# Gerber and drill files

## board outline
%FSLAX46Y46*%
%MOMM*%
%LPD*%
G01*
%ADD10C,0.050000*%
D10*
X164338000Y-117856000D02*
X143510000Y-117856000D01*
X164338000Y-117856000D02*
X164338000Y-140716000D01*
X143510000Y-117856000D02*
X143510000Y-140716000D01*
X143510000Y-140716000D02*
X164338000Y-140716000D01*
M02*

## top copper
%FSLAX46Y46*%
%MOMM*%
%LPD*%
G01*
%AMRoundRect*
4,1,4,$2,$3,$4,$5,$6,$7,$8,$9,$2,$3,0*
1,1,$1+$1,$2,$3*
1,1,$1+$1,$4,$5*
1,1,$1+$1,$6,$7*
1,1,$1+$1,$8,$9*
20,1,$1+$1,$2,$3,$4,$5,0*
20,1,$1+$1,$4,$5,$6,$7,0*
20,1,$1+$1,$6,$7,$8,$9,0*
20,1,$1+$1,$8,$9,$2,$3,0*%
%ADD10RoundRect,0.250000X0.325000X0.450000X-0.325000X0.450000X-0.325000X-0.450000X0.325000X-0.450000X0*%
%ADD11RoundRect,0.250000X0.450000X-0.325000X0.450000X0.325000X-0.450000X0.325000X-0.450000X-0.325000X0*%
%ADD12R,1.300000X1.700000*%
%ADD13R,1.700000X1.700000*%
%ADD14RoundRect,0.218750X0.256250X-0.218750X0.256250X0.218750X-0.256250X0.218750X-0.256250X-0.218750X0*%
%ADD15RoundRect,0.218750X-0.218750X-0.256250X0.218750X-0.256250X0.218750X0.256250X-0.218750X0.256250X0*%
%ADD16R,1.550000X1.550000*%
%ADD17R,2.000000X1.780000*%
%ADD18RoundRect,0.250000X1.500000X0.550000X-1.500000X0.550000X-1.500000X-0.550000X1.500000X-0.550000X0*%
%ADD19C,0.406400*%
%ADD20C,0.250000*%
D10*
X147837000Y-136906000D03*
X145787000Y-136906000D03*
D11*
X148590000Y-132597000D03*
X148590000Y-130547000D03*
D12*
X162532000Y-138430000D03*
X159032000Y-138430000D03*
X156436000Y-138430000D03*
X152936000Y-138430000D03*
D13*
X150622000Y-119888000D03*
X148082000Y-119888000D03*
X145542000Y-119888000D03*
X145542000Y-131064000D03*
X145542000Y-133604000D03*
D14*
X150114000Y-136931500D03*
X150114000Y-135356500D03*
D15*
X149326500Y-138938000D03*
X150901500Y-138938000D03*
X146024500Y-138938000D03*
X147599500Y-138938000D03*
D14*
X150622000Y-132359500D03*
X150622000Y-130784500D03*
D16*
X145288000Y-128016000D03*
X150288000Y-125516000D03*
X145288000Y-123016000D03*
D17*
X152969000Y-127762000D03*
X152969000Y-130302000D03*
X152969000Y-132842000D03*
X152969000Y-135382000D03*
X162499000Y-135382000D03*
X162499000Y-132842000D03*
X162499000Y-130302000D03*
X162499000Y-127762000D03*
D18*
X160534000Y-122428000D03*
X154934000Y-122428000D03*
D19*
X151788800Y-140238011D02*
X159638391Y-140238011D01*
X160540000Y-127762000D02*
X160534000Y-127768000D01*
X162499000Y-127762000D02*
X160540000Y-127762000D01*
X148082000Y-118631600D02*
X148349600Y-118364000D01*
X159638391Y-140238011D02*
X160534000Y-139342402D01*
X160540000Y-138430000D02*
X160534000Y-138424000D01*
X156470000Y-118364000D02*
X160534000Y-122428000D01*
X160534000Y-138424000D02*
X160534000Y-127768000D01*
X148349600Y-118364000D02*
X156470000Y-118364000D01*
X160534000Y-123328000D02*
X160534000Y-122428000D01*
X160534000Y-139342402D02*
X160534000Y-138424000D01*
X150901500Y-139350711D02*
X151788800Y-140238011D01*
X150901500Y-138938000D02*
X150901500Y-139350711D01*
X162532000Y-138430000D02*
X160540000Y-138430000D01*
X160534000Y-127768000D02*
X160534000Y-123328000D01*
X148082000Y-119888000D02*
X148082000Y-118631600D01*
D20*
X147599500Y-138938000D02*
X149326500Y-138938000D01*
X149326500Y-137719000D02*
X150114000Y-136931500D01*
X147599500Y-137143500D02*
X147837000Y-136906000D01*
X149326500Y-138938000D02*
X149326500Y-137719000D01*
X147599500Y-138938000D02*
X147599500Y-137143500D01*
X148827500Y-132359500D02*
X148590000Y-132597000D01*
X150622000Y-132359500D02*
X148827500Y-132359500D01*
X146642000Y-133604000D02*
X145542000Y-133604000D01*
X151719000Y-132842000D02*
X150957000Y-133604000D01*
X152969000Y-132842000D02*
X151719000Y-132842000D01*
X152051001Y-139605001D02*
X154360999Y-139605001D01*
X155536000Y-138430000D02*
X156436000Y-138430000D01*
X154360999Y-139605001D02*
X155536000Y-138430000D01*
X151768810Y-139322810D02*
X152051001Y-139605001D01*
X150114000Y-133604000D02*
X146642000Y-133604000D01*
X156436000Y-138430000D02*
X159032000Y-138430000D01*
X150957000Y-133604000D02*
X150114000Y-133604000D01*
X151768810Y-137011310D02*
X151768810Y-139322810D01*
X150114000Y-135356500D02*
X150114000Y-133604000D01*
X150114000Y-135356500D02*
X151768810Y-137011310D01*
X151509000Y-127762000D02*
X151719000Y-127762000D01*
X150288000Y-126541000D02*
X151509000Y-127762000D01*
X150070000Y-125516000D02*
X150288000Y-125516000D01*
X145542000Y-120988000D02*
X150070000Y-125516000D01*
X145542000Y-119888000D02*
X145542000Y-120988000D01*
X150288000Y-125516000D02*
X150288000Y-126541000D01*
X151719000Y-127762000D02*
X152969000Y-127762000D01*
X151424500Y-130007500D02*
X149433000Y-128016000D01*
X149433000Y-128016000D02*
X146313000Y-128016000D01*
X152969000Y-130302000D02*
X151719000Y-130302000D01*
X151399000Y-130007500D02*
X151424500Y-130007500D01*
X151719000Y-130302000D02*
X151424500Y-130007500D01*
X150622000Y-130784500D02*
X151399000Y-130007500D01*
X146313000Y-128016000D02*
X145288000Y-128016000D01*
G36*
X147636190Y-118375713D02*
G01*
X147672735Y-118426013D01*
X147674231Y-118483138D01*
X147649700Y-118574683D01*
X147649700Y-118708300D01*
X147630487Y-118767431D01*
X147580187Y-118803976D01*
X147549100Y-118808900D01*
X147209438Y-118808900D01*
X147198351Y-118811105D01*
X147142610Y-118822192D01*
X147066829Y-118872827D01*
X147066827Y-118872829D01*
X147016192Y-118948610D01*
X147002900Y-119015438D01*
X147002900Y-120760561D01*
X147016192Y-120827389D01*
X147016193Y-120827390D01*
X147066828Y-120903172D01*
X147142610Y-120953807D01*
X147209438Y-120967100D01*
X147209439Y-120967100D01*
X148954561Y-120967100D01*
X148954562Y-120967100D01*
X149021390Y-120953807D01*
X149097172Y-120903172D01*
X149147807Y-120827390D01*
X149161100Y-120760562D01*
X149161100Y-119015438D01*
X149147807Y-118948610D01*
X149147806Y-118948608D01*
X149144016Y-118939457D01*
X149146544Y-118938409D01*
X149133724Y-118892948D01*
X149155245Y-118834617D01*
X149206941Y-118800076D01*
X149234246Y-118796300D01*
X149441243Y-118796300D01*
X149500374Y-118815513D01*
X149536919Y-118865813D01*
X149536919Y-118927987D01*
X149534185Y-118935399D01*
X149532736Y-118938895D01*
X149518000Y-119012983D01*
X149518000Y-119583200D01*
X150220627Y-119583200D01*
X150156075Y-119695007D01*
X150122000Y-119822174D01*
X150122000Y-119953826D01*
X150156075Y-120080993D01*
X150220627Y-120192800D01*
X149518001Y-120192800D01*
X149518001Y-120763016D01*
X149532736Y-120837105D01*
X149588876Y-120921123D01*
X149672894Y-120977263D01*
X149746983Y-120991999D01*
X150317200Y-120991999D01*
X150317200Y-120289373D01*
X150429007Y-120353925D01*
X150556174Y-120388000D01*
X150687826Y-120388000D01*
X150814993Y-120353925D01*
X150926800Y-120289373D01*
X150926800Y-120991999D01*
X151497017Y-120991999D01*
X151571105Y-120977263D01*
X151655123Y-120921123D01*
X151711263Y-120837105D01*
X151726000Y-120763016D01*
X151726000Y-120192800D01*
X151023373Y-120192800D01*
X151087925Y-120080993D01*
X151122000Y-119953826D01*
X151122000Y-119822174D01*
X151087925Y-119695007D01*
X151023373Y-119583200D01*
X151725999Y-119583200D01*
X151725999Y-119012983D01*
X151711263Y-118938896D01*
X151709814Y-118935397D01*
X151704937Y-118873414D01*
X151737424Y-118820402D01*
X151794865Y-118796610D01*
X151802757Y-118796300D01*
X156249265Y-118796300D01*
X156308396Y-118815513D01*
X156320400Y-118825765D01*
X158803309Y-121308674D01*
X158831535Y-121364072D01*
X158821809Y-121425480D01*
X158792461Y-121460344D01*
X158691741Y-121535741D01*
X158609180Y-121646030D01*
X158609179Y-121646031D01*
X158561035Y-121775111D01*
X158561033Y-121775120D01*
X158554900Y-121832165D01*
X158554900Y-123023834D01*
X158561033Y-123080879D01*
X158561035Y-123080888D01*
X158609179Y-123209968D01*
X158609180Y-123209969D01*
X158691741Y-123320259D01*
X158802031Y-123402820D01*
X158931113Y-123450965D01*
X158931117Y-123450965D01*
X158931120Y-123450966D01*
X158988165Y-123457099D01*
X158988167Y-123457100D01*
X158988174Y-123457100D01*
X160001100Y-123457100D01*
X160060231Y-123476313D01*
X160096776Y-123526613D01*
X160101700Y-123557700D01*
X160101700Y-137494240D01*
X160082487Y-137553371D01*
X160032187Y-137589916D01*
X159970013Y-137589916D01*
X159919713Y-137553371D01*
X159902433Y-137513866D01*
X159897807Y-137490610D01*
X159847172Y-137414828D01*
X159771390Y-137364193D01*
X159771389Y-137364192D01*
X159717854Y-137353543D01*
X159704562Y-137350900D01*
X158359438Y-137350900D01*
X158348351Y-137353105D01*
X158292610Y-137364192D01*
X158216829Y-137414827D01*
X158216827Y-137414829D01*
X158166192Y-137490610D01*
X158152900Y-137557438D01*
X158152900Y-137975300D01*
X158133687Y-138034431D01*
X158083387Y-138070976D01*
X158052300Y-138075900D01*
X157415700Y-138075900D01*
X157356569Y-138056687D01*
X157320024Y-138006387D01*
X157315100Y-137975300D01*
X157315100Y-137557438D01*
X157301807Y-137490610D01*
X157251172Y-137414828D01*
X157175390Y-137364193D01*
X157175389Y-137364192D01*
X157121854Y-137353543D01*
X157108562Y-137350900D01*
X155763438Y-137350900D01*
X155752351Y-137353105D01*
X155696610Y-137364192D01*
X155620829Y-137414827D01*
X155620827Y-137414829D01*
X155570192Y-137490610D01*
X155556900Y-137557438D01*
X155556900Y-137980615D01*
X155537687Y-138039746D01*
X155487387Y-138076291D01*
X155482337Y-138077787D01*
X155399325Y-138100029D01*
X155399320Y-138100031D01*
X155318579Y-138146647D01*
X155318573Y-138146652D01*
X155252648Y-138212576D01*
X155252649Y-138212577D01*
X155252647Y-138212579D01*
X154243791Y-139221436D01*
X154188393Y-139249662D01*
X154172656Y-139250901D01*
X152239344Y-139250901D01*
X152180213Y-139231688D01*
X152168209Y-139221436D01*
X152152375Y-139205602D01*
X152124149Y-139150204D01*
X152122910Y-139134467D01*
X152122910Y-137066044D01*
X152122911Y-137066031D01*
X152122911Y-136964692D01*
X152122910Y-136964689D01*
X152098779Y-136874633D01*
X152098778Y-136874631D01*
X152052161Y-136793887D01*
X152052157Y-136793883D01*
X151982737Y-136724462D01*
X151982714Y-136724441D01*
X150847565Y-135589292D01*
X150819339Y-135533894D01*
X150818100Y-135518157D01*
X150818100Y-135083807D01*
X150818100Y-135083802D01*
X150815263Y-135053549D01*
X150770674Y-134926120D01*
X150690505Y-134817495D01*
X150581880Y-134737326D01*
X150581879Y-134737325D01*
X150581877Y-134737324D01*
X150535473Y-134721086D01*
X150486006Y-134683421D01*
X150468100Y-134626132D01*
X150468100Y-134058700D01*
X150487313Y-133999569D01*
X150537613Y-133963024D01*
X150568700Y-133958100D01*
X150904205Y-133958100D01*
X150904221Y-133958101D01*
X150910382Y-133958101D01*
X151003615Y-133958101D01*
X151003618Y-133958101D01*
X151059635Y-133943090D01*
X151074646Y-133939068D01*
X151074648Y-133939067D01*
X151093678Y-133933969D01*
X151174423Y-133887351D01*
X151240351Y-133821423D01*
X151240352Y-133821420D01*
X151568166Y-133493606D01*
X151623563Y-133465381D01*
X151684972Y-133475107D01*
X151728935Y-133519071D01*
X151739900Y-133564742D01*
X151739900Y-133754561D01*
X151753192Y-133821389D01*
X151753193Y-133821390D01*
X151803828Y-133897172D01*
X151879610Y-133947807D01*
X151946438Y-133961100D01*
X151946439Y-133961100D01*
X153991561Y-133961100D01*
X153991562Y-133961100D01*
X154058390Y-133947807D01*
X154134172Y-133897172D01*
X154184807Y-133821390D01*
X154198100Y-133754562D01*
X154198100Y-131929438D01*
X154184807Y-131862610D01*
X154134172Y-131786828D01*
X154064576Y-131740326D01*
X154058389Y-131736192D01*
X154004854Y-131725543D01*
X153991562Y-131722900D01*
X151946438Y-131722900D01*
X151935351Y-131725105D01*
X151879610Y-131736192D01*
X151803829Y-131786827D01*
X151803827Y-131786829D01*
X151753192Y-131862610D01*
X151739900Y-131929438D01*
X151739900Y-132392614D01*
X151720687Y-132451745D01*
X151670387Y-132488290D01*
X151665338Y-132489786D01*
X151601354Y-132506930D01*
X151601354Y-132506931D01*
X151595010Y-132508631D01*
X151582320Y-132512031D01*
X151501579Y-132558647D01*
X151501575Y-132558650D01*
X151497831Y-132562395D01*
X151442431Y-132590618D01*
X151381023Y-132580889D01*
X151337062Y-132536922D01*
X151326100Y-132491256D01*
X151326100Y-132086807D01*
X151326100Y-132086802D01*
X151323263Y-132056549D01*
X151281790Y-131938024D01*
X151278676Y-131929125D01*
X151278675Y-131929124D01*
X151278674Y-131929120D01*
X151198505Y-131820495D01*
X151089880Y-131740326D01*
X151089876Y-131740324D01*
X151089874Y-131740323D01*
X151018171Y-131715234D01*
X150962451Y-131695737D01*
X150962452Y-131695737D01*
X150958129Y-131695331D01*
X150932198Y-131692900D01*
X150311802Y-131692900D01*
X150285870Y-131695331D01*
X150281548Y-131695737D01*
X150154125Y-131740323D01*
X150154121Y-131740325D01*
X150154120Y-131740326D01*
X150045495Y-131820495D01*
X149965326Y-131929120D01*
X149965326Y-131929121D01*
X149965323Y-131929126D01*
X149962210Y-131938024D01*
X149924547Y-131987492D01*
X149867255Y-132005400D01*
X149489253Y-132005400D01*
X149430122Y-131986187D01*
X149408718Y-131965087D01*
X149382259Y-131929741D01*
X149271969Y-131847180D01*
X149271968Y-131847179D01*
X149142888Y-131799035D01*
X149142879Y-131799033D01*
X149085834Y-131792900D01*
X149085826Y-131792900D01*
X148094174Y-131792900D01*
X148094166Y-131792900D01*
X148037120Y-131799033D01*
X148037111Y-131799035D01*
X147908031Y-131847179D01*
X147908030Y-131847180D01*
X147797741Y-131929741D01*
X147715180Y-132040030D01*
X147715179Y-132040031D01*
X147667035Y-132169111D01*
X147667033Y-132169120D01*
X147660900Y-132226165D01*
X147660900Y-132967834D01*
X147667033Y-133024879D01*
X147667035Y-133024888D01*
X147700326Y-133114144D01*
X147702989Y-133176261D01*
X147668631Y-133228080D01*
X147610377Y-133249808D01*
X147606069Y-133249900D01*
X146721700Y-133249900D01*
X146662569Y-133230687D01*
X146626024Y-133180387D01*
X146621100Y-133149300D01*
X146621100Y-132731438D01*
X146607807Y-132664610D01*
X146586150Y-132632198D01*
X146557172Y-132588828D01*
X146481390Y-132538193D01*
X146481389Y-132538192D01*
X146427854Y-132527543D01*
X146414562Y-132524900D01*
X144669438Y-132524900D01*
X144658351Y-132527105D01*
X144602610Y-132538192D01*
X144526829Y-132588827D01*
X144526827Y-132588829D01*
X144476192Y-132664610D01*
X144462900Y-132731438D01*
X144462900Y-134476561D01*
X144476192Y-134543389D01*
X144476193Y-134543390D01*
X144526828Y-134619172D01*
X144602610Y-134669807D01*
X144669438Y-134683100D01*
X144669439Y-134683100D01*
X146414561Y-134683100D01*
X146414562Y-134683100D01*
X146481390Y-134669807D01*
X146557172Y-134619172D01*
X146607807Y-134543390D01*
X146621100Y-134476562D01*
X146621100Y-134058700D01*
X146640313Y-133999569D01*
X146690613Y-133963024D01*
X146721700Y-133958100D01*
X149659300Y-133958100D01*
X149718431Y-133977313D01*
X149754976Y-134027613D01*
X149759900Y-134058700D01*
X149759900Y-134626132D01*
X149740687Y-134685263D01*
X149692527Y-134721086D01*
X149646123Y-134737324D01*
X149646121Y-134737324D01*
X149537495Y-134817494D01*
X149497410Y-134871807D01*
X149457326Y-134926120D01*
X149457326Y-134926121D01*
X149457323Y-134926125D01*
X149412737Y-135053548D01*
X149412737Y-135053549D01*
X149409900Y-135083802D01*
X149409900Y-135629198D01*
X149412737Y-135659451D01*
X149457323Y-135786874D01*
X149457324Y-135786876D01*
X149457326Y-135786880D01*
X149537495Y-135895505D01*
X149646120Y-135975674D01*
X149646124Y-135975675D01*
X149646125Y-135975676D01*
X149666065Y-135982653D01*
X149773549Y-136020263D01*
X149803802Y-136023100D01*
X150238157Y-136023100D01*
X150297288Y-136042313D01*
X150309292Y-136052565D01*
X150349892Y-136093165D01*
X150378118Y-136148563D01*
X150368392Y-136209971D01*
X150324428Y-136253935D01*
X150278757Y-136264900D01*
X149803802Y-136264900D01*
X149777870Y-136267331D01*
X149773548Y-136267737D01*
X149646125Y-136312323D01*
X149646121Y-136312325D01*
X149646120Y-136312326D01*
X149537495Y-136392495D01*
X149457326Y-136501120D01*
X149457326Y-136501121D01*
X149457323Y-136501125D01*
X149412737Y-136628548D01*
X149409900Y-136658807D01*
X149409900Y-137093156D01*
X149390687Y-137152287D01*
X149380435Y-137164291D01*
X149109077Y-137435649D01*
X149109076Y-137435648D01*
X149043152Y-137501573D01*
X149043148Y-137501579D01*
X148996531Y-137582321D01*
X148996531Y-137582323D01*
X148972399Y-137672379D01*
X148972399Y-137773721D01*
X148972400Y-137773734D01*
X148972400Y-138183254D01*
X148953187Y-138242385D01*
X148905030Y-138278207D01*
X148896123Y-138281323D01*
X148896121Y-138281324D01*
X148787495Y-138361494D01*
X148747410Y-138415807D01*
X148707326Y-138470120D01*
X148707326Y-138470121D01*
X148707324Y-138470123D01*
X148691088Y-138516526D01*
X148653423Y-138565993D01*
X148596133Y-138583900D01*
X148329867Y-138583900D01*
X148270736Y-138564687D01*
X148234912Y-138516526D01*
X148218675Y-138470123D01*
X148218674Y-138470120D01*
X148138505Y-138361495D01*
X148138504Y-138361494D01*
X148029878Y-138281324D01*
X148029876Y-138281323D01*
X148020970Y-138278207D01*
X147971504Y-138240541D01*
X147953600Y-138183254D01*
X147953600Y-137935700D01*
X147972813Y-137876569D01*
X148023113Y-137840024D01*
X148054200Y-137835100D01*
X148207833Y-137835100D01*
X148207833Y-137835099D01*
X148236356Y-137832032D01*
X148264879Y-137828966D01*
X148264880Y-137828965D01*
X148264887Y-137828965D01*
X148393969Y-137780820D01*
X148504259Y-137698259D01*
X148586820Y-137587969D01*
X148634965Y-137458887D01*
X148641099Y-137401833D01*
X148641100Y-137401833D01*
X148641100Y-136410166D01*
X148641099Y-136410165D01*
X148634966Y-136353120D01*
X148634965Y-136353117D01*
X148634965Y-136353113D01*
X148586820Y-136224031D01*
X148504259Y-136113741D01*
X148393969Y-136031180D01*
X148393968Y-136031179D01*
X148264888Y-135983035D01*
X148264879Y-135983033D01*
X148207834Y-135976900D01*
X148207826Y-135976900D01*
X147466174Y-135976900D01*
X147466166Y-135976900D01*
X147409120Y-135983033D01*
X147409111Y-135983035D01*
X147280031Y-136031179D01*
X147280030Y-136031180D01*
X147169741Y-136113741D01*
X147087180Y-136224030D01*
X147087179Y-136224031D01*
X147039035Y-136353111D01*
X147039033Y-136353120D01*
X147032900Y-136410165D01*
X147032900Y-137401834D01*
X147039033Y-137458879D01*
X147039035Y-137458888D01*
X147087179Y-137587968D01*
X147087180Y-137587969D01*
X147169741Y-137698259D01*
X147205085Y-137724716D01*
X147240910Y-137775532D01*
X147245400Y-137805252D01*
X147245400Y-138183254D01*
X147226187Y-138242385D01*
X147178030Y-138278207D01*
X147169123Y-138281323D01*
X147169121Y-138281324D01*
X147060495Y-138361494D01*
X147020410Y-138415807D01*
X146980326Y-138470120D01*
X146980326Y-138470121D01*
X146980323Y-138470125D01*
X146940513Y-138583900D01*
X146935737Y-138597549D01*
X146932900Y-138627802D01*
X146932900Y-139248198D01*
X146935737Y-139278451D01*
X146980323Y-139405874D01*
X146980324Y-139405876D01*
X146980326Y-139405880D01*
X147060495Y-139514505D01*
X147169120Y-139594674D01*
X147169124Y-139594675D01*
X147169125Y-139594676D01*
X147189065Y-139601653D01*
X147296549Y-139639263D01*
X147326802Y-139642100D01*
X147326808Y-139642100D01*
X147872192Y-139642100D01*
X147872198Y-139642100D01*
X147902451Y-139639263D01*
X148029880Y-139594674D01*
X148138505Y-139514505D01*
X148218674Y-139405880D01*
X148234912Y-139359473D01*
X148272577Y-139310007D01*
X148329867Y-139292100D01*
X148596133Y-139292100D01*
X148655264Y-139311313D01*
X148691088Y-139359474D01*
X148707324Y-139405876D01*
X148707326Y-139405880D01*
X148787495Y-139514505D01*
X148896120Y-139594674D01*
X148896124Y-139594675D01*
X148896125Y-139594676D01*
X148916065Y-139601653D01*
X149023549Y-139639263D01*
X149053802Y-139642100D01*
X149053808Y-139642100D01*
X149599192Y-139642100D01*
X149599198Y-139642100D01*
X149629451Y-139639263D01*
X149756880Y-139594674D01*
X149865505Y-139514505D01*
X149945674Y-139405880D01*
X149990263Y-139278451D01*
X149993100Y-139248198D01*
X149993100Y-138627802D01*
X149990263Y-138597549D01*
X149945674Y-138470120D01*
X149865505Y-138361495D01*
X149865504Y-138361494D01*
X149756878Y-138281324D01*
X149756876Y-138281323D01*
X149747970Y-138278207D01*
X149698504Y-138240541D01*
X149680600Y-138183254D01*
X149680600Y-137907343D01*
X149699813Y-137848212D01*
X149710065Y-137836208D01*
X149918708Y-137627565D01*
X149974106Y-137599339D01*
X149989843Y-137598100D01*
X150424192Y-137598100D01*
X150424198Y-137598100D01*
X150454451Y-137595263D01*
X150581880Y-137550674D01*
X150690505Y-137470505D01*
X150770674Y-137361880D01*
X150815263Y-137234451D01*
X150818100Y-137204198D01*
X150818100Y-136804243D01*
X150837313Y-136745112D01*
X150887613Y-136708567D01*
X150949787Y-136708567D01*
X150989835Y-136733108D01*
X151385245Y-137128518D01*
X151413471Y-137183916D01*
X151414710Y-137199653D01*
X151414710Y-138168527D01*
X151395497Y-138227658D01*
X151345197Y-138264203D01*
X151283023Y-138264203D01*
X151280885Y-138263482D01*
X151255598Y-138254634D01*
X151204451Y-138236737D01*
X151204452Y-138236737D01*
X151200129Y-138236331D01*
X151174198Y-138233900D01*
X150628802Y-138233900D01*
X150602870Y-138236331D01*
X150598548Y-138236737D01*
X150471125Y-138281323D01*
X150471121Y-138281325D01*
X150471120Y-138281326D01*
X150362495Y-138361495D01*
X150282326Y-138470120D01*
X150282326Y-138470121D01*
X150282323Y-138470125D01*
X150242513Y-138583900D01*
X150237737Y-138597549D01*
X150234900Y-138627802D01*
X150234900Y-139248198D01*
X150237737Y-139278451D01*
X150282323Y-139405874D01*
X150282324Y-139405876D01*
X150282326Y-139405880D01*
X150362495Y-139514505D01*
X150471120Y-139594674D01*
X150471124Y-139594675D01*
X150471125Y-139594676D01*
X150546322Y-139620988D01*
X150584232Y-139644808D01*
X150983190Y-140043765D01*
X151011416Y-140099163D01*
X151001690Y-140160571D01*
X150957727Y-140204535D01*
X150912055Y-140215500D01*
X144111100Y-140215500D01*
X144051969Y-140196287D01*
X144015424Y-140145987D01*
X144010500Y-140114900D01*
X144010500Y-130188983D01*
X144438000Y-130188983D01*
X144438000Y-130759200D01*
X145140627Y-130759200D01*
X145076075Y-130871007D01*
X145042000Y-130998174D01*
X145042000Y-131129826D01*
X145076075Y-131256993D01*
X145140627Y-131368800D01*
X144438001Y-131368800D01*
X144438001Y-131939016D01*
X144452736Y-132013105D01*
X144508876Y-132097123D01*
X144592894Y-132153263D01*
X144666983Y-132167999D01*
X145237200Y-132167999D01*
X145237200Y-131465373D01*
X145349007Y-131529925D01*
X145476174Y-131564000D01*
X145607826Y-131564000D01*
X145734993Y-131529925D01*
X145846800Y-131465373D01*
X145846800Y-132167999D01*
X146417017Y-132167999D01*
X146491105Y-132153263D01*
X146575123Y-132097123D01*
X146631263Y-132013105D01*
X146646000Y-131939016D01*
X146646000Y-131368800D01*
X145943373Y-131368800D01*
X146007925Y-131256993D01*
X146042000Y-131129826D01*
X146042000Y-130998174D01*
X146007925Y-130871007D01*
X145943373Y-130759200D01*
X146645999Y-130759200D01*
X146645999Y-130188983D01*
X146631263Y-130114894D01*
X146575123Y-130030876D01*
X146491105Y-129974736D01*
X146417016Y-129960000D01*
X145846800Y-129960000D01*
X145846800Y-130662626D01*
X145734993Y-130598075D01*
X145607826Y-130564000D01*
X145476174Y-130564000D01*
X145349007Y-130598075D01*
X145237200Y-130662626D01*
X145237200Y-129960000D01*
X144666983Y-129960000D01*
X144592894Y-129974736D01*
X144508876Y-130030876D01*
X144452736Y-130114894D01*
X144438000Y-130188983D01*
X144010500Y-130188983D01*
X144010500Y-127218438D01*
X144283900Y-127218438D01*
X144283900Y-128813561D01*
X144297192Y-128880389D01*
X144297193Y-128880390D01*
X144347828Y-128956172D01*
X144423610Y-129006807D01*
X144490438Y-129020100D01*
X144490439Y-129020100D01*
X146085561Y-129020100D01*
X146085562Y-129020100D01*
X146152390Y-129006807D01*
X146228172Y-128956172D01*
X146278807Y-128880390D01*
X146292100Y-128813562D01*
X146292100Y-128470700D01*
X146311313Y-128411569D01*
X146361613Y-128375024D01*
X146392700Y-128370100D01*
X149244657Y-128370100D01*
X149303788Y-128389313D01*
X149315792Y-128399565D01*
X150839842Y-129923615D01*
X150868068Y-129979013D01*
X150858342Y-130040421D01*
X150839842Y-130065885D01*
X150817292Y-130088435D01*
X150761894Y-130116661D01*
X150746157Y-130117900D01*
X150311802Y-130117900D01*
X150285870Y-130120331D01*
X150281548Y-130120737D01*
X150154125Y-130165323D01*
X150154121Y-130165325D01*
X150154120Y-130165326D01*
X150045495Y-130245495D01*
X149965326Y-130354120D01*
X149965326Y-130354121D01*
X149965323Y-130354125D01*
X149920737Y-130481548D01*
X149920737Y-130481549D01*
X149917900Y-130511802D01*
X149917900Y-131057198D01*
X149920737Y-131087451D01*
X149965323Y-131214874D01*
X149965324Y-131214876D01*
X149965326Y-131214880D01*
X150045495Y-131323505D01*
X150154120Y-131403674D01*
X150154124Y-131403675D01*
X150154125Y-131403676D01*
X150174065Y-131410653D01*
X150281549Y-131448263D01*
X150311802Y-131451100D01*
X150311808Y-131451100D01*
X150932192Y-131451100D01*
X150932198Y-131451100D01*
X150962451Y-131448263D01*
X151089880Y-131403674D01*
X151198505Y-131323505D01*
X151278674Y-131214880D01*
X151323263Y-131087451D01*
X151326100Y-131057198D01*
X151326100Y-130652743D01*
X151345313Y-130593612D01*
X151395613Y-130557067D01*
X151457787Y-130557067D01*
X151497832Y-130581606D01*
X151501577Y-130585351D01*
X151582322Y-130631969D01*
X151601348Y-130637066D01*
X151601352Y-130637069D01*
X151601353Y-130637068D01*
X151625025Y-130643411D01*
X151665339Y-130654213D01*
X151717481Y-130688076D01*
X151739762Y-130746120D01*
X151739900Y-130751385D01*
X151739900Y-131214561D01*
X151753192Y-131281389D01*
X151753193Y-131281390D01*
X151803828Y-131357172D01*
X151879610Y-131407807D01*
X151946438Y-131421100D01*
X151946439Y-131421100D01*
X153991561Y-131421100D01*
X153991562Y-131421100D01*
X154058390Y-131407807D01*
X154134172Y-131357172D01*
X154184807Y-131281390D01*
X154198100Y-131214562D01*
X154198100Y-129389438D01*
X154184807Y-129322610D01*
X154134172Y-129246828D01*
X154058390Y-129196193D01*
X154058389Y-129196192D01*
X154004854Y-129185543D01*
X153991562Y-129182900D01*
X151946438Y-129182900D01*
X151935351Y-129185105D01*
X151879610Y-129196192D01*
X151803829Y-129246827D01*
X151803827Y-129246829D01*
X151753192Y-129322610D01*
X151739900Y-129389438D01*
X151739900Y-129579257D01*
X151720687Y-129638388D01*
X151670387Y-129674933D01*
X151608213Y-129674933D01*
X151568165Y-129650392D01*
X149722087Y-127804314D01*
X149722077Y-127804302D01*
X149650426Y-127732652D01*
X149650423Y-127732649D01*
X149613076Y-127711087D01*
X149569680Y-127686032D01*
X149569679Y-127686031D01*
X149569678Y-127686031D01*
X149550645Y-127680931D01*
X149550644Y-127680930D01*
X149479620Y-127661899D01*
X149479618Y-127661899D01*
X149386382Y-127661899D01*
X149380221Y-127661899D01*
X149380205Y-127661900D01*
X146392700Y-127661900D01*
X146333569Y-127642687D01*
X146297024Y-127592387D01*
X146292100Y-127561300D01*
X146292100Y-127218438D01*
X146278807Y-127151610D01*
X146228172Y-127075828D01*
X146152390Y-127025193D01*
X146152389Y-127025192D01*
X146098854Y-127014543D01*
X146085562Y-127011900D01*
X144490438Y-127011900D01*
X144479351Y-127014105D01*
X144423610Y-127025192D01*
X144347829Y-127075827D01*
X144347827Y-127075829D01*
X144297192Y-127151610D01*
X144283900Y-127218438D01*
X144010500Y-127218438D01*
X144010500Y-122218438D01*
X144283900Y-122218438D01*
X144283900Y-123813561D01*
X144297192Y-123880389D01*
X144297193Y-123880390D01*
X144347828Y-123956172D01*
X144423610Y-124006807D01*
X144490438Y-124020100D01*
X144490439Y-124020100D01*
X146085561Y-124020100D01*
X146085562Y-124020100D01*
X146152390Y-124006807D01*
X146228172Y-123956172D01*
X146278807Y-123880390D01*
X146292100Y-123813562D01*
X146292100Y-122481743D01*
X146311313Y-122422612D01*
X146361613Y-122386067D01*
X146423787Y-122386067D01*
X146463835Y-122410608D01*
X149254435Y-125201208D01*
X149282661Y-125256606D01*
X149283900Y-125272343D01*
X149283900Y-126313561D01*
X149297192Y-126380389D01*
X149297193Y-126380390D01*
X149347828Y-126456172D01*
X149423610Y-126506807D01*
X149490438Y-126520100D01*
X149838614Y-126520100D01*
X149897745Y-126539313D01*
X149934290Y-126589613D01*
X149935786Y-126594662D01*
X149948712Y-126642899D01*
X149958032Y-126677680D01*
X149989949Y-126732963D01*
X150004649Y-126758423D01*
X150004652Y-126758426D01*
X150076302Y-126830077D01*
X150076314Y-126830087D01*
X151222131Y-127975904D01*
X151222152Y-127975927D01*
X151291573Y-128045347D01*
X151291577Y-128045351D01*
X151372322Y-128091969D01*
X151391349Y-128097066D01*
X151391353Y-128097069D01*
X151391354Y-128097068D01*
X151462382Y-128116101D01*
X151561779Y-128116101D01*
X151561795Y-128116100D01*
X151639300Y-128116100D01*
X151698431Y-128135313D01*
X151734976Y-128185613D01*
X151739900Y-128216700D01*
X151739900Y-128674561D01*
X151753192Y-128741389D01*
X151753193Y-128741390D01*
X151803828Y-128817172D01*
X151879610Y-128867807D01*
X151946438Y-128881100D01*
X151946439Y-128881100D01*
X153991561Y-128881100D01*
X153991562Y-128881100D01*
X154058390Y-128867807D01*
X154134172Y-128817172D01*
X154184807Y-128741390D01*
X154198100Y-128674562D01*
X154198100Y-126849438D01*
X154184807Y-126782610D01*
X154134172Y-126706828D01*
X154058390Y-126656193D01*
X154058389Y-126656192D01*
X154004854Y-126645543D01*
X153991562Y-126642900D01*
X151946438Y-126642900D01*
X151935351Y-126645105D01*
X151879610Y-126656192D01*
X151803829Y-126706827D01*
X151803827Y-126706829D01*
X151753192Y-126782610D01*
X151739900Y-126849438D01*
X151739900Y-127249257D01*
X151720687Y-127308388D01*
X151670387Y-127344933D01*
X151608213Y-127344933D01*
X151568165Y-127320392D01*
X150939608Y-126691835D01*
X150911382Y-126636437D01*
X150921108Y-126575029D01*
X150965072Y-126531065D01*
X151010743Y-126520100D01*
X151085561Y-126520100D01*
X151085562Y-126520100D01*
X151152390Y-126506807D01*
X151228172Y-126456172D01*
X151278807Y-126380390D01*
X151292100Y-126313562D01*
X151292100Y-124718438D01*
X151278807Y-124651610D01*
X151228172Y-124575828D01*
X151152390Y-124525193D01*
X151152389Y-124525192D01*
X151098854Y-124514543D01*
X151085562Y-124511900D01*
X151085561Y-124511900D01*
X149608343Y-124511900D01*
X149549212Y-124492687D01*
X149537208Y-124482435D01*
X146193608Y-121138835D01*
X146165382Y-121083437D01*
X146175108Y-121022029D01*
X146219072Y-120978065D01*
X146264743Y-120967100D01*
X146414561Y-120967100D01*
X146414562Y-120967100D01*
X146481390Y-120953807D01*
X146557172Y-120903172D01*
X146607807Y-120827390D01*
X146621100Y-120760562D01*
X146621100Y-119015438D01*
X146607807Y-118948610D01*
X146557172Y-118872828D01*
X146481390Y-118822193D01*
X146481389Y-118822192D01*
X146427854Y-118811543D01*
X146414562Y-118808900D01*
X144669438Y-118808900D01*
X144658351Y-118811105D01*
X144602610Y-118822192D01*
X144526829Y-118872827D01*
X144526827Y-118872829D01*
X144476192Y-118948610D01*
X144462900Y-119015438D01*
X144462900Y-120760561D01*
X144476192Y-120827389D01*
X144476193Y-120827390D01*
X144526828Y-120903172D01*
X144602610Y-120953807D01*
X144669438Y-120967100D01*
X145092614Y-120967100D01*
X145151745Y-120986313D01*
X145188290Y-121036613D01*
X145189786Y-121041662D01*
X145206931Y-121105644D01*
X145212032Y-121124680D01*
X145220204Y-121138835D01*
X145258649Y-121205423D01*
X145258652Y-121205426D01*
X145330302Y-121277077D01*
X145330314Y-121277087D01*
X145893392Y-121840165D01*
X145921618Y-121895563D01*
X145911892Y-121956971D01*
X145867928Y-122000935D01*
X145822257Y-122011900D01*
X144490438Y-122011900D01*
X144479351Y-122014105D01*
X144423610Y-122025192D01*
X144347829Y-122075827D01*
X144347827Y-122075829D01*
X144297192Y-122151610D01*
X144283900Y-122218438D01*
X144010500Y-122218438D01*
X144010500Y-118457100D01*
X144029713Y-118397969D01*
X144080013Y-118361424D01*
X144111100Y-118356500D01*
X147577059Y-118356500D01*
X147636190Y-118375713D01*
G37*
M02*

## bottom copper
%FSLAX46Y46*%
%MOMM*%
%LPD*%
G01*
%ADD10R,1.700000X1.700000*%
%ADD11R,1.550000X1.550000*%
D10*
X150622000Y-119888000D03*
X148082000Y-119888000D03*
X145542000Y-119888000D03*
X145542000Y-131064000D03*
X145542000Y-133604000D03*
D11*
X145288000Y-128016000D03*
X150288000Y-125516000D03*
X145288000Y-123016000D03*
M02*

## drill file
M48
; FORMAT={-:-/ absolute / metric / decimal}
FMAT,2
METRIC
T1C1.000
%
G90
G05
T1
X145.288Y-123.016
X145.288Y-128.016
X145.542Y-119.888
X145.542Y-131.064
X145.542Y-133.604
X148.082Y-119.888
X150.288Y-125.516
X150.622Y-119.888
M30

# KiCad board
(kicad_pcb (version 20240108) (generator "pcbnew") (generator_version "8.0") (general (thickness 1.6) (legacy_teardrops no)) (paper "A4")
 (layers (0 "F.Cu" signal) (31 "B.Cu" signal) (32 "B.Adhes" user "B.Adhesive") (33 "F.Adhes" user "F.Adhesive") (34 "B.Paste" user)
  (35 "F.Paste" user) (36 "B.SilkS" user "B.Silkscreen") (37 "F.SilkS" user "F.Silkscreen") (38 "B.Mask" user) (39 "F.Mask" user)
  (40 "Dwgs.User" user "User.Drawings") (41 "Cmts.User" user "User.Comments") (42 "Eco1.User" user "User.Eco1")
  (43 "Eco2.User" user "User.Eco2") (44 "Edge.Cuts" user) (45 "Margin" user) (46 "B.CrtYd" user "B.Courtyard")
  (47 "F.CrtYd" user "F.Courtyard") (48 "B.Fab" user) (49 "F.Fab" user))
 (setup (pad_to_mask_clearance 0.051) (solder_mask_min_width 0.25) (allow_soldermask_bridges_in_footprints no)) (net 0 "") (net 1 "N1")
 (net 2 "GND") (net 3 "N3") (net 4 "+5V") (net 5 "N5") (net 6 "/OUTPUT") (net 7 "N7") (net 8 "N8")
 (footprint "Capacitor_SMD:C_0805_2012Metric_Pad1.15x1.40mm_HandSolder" (layer "F.Cu") (at 146.812 136.906 180)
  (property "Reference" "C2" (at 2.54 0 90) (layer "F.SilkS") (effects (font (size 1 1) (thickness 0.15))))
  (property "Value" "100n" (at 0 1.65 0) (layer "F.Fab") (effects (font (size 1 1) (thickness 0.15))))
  (pad "1" smd roundrect (at -1.025 0 180) (size 1.15 1.4) (layers "F.Cu" "F.Paste" "F.Mask") (roundrect_rratio 0.217391) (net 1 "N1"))
  (pad "2" smd roundrect (at 1.025 0 180) (size 1.15 1.4) (layers "F.Cu" "F.Paste" "F.Mask") (roundrect_rratio 0.217391) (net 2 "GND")))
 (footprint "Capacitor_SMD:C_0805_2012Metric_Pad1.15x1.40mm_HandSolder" (layer "F.Cu") (at 148.59 131.572 90)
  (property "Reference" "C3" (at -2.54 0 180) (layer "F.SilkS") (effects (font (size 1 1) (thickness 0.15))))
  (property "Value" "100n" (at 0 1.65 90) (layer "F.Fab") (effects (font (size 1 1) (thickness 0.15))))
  (pad "1" smd roundrect (at -1.025 0 90) (size 1.15 1.4) (layers "F.Cu" "F.Paste" "F.Mask") (roundrect_rratio 0.217391) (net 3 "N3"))
  (pad "2" smd roundrect (at 1.025 0 90) (size 1.15 1.4) (layers "F.Cu" "F.Paste" "F.Mask") (roundrect_rratio 0.217391) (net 2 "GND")))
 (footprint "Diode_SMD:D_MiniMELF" (layer "F.Cu") (at 160.782 138.43 180)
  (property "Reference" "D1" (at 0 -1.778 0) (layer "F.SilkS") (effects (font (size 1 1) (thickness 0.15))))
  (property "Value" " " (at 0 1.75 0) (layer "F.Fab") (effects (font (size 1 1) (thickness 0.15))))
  (pad "1" smd rect (at -1.75 0 180) (size 1.3 1.7) (layers "F.Cu" "F.Paste" "F.Mask") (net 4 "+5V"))
  (pad "2" smd rect (at 1.75 0 180) (size 1.3 1.7) (layers "F.Cu" "F.Paste" "F.Mask") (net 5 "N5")))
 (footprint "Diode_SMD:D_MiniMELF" (layer "F.Cu") (at 154.686 138.43 180)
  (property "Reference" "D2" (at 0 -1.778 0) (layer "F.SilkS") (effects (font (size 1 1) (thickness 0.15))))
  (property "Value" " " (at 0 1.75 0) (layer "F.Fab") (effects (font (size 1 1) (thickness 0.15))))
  (pad "1" smd rect (at -1.75 0 180) (size 1.3 1.7) (layers "F.Cu" "F.Paste" "F.Mask") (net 5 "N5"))
  (pad "2" smd rect (at 1.75 0 180) (size 1.3 1.7) (layers "F.Cu" "F.Paste" "F.Mask") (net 2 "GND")))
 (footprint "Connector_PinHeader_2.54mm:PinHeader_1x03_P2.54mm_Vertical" (layer "F.Cu") (at 150.622 119.888 -90)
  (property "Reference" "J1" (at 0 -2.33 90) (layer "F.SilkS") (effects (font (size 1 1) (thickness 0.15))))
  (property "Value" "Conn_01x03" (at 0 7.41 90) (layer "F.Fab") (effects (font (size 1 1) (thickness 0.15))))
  (pad "1" thru_hole rect (at 0 0 270) (size 1.7 1.7) (drill 1) (layers "*.Cu" "*.Mask") (remove_unused_layers no) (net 2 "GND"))
  (pad "2" thru_hole rect (at 0 2.54 270) (size 1.7 1.7) (drill 1) (layers "*.Cu" "*.Mask") (remove_unused_layers no) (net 4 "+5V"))
  (pad "3" thru_hole rect (at 0 5.08 270) (size 1.7 1.7) (drill 1) (layers "*.Cu" "*.Mask") (remove_unused_layers no) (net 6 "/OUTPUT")))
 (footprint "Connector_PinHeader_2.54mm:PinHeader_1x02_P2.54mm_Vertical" (layer "F.Cu") (at 145.542 131.064)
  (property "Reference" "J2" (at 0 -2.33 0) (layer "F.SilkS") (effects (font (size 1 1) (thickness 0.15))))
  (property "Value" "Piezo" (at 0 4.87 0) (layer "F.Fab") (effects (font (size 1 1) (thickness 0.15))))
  (pad "1" thru_hole rect (at 0 0) (size 1.7 1.7) (drill 1) (layers "*.Cu" "*.Mask") (remove_unused_layers no) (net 2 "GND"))
  (pad "2" thru_hole rect (at 0 2.54) (size 1.7 1.7) (drill 1) (layers "*.Cu" "*.Mask") (remove_unused_layers no) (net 5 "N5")))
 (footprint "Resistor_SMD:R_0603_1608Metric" (layer "F.Cu") (at 150.114 136.144 90)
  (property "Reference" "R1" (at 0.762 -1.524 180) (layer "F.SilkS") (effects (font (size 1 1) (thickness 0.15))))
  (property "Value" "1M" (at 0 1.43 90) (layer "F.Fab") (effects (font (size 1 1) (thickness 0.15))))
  (pad "1" smd roundrect (at -0.7875 0 90) (size 0.875 0.95) (layers "F.Cu" "F.Paste" "F.Mask") (roundrect_rratio 0.25) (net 1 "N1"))
  (pad "2" smd roundrect (at 0.7875 0 90) (size 0.875 0.95) (layers "F.Cu" "F.Paste" "F.Mask") (roundrect_rratio 0.25) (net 5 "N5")))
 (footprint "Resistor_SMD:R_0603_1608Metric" (layer "F.Cu") (at 150.114 138.938)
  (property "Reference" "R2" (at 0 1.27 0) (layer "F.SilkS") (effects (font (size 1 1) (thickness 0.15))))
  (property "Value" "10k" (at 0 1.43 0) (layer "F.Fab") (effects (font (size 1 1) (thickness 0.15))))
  (pad "1" smd roundrect (at -0.7875 0) (size 0.875 0.95) (layers "F.Cu" "F.Paste" "F.Mask") (roundrect_rratio 0.25) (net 1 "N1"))
  (pad "2" smd roundrect (at 0.7875 0) (size 0.875 0.95) (layers "F.Cu" "F.Paste" "F.Mask") (roundrect_rratio 0.25) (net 4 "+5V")))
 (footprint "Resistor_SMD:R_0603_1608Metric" (layer "F.Cu") (at 146.812 138.938)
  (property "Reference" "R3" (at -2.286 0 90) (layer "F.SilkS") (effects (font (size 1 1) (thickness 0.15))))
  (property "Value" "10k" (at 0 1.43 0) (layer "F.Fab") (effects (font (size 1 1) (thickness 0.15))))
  (pad "1" smd roundrect (at -0.7875 0) (size 0.875 0.95) (layers "F.Cu" "F.Paste" "F.Mask") (roundrect_rratio 0.25) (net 2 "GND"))
  (pad "2" smd roundrect (at 0.7875 0) (size 0.875 0.95) (layers "F.Cu" "F.Paste" "F.Mask") (roundrect_rratio 0.25) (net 1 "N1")))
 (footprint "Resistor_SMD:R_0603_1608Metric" (layer "F.Cu") (at 150.622 131.572 90)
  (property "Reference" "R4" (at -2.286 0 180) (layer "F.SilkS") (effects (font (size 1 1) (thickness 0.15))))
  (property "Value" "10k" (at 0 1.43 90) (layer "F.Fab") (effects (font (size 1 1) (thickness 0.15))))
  (pad "1" smd roundrect (at -0.7875 0 90) (size 0.875 0.95) (layers "F.Cu" "F.Paste" "F.Mask") (roundrect_rratio 0.25) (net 3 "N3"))
  (pad "2" smd roundrect (at 0.7875 0 90) (size 0.875 0.95) (layers "F.Cu" "F.Paste" "F.Mask") (roundrect_rratio 0.25) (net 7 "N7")))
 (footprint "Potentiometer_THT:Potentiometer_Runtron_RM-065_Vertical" (layer "F.Cu") (at 145.288 128.016 90)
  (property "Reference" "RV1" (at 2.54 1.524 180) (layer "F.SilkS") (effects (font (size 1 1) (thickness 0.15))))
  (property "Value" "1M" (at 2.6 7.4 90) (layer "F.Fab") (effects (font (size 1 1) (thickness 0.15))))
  (pad "1" thru_hole rect (at 0 0 90) (size 1.55 1.55) (drill 1) (layers "*.Cu" "*.Mask") (remove_unused_layers no) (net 7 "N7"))
  (pad "2" thru_hole rect (at 2.5 5 90) (size 1.55 1.55) (drill 1) (layers "*.Cu" "*.Mask") (remove_unused_layers no) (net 6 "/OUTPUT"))
  (pad "3" thru_hole rect (at 5 0 90) (size 1.55 1.55) (drill 1) (layers "*.Cu" "*.Mask") (remove_unused_layers no) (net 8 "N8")))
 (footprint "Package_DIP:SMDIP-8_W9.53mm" (layer "F.Cu") (at 157.734 131.572)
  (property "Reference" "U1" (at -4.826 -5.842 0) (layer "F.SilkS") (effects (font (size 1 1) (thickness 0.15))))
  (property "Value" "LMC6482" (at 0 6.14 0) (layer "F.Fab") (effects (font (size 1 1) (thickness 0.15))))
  (pad "1" smd rect (at -4.765 -3.81) (size 2 1.78) (layers "F.Cu" "F.Paste" "F.Mask") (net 6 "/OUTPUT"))
  (pad "2" smd rect (at -4.765 -1.27) (size 2 1.78) (layers "F.Cu" "F.Paste" "F.Mask") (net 7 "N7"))
  (pad "3" smd rect (at -4.765 1.27) (size 2 1.78) (layers "F.Cu" "F.Paste" "F.Mask") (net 5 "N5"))
  (pad "4" smd rect (at -4.765 3.81) (size 2 1.78) (layers "F.Cu" "F.Paste" "F.Mask") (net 2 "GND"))
  (pad "5" smd rect (at 4.765 3.81) (size 2 1.78) (layers "F.Cu" "F.Paste" "F.Mask"))
  (pad "6" smd rect (at 4.765 1.27) (size 2 1.78) (layers "F.Cu" "F.Paste" "F.Mask"))
  (pad "7" smd rect (at 4.765 -1.27) (size 2 1.78) (layers "F.Cu" "F.Paste" "F.Mask"))
  (pad "8" smd rect (at 4.765 -3.81) (size 2 1.78) (layers "F.Cu" "F.Paste" "F.Mask") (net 4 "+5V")))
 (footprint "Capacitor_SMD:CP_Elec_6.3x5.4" (layer "F.Cu") (at 157.734 122.428 180)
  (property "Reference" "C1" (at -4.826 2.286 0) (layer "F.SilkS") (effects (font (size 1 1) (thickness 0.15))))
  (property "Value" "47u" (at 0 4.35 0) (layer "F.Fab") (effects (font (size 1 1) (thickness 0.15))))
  (pad "1" smd roundrect (at -2.8 0 180) (size 3.5 1.6) (layers "F.Cu" "F.Paste" "F.Mask") (roundrect_rratio 0.15625) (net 4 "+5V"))
  (pad "2" smd roundrect (at 2.8 0 180) (size 3.5 1.6) (layers "F.Cu" "F.Paste" "F.Mask") (roundrect_rratio 0.15625) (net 2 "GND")))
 (gr_line (start 164.338 117.856) (end 143.51 117.856) (stroke (width 0.05) (type solid)) (layer "Edge.Cuts"))
 (gr_line (start 164.338 117.856) (end 164.338 140.716) (stroke (width 0.05) (type solid)) (layer "Edge.Cuts"))
 (gr_line (start 143.51 117.856) (end 143.51 140.716) (stroke (width 0.05) (type solid)) (layer "Edge.Cuts"))
 (gr_line (start 143.51 140.716) (end 164.338 140.716) (stroke (width 0.05) (type solid)) (layer "Edge.Cuts"))
 (segment (start 151.7888 140.238011) (end 159.638391 140.238011) (width 0.4064) (layer "F.Cu") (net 4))
 (segment (start 160.54 127.762) (end 160.534 127.768) (width 0.4064) (layer "F.Cu") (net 4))
 (segment (start 162.499 127.762) (end 160.54 127.762) (width 0.4064) (layer "F.Cu") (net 4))
 (segment (start 148.082 118.6316) (end 148.3496 118.364) (width 0.4064) (layer "F.Cu") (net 4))
 (segment (start 159.638391 140.238011) (end 160.534 139.342402) (width 0.4064) (layer "F.Cu") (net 4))
 (segment (start 160.54 138.43) (end 160.534 138.424) (width 0.4064) (layer "F.Cu") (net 4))
 (segment (start 156.47 118.364) (end 160.534 122.428) (width 0.4064) (layer "F.Cu") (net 4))
 (segment (start 160.534 138.424) (end 160.534 127.768) (width 0.4064) (layer "F.Cu") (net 4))
 (segment (start 148.3496 118.364) (end 156.47 118.364) (width 0.4064) (layer "F.Cu") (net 4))
 (segment (start 160.534 123.328) (end 160.534 122.428) (width 0.4064) (layer "F.Cu") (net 4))
 (segment (start 160.534 139.342402) (end 160.534 138.424) (width 0.4064) (layer "F.Cu") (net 4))
 (segment (start 150.9015 139.350711) (end 151.7888 140.238011) (width 0.4064) (layer "F.Cu") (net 4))
 (segment (start 150.9015 138.938) (end 150.9015 139.350711) (width 0.4064) (layer "F.Cu") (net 4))
 (segment (start 162.532 138.43) (end 160.54 138.43) (width 0.4064) (layer "F.Cu") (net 4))
 (segment (start 160.534 127.768) (end 160.534 123.328) (width 0.4064) (layer "F.Cu") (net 4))
 (segment (start 148.082 119.888) (end 148.082 118.6316) (width 0.4064) (layer "F.Cu") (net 4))
 (segment (start 147.5995 138.938) (end 149.3265 138.938) (width 0.25) (layer "F.Cu") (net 1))
 (segment (start 149.3265 137.719) (end 150.114 136.9315) (width 0.25) (layer "F.Cu") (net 1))
 (segment (start 147.5995 137.1435) (end 147.837 136.906) (width 0.25) (layer "F.Cu") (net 1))
 (segment (start 149.3265 138.938) (end 149.3265 137.719) (width 0.25) (layer "F.Cu") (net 1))
 (segment (start 147.5995 138.938) (end 147.5995 137.1435) (width 0.25) (layer "F.Cu") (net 1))
 (segment (start 148.8275 132.3595) (end 148.59 132.597) (width 0.25) (layer "F.Cu") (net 3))
 (segment (start 150.622 132.3595) (end 148.8275 132.3595) (width 0.25) (layer "F.Cu") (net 3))
 (segment (start 146.642 133.604) (end 145.542 133.604) (width 0.25) (layer "F.Cu") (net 5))
 (segment (start 151.719 132.842) (end 150.957 133.604) (width 0.25) (layer "F.Cu") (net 5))
 (segment (start 152.969 132.842) (end 151.719 132.842) (width 0.25) (layer "F.Cu") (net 5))
 (segment (start 152.051001 139.605001) (end 154.360999 139.605001) (width 0.25) (layer "F.Cu") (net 5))
 (segment (start 155.536 138.43) (end 156.436 138.43) (width 0.25) (layer "F.Cu") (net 5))
 (segment (start 154.360999 139.605001) (end 155.536 138.43) (width 0.25) (layer "F.Cu") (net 5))
 (segment (start 151.76881 139.32281) (end 152.051001 139.605001) (width 0.25) (layer "F.Cu") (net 5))
 (segment (start 150.114 133.604) (end 146.642 133.604) (width 0.25) (layer "F.Cu") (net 5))
 (segment (start 156.436 138.43) (end 159.032 138.43) (width 0.25) (layer "F.Cu") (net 5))
 (segment (start 150.957 133.604) (end 150.114 133.604) (width 0.25) (layer "F.Cu") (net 5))
 (segment (start 151.76881 137.01131) (end 151.76881 139.32281) (width 0.25) (layer "F.Cu") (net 5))
 (segment (start 150.114 135.3565) (end 150.114 133.604) (width 0.25) (layer "F.Cu") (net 5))
 (segment (start 150.114 135.3565) (end 151.76881 137.01131) (width 0.25) (layer "F.Cu") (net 5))
 (segment (start 151.509 127.762) (end 151.719 127.762) (width 0.25) (layer "F.Cu") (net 6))
 (segment (start 150.288 126.541) (end 151.509 127.762) (width 0.25) (layer "F.Cu") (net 6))
 (segment (start 150.07 125.516) (end 150.288 125.516) (width 0.25) (layer "F.Cu") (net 6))
 (segment (start 145.542 120.988) (end 150.07 125.516) (width 0.25) (layer "F.Cu") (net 6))
 (segment (start 145.542 119.888) (end 145.542 120.988) (width 0.25) (layer "F.Cu") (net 6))
 (segment (start 150.288 125.516) (end 150.288 126.541) (width 0.25) (layer "F.Cu") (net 6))
 (segment (start 151.719 127.762) (end 152.969 127.762) (width 0.25) (layer "F.Cu") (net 6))
 (segment (start 151.4245 130.0075) (end 149.433 128.016) (width 0.25) (layer "F.Cu") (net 7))
 (segment (start 149.433 128.016) (end 146.313 128.016) (width 0.25) (layer "F.Cu") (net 7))
 (segment (start 152.969 130.302) (end 151.719 130.302) (width 0.25) (layer "F.Cu") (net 7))
 (segment (start 151.399 130.0075) (end 151.4245 130.0075) (width 0.25) (layer "F.Cu") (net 7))
 (segment (start 151.719 130.302) (end 151.4245 130.0075) (width 0.25) (layer "F.Cu") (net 7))
 (segment (start 150.622 130.7845) (end 151.399 130.0075) (width 0.25) (layer "F.Cu") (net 7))
 (segment (start 146.313 128.016) (end 145.288 128.016) (width 0.25) (layer "F.Cu") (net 7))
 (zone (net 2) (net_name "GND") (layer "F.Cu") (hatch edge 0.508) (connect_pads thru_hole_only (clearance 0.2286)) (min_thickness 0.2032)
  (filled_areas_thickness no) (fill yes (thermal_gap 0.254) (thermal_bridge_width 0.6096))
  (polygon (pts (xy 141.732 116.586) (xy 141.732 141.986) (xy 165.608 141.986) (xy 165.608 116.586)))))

